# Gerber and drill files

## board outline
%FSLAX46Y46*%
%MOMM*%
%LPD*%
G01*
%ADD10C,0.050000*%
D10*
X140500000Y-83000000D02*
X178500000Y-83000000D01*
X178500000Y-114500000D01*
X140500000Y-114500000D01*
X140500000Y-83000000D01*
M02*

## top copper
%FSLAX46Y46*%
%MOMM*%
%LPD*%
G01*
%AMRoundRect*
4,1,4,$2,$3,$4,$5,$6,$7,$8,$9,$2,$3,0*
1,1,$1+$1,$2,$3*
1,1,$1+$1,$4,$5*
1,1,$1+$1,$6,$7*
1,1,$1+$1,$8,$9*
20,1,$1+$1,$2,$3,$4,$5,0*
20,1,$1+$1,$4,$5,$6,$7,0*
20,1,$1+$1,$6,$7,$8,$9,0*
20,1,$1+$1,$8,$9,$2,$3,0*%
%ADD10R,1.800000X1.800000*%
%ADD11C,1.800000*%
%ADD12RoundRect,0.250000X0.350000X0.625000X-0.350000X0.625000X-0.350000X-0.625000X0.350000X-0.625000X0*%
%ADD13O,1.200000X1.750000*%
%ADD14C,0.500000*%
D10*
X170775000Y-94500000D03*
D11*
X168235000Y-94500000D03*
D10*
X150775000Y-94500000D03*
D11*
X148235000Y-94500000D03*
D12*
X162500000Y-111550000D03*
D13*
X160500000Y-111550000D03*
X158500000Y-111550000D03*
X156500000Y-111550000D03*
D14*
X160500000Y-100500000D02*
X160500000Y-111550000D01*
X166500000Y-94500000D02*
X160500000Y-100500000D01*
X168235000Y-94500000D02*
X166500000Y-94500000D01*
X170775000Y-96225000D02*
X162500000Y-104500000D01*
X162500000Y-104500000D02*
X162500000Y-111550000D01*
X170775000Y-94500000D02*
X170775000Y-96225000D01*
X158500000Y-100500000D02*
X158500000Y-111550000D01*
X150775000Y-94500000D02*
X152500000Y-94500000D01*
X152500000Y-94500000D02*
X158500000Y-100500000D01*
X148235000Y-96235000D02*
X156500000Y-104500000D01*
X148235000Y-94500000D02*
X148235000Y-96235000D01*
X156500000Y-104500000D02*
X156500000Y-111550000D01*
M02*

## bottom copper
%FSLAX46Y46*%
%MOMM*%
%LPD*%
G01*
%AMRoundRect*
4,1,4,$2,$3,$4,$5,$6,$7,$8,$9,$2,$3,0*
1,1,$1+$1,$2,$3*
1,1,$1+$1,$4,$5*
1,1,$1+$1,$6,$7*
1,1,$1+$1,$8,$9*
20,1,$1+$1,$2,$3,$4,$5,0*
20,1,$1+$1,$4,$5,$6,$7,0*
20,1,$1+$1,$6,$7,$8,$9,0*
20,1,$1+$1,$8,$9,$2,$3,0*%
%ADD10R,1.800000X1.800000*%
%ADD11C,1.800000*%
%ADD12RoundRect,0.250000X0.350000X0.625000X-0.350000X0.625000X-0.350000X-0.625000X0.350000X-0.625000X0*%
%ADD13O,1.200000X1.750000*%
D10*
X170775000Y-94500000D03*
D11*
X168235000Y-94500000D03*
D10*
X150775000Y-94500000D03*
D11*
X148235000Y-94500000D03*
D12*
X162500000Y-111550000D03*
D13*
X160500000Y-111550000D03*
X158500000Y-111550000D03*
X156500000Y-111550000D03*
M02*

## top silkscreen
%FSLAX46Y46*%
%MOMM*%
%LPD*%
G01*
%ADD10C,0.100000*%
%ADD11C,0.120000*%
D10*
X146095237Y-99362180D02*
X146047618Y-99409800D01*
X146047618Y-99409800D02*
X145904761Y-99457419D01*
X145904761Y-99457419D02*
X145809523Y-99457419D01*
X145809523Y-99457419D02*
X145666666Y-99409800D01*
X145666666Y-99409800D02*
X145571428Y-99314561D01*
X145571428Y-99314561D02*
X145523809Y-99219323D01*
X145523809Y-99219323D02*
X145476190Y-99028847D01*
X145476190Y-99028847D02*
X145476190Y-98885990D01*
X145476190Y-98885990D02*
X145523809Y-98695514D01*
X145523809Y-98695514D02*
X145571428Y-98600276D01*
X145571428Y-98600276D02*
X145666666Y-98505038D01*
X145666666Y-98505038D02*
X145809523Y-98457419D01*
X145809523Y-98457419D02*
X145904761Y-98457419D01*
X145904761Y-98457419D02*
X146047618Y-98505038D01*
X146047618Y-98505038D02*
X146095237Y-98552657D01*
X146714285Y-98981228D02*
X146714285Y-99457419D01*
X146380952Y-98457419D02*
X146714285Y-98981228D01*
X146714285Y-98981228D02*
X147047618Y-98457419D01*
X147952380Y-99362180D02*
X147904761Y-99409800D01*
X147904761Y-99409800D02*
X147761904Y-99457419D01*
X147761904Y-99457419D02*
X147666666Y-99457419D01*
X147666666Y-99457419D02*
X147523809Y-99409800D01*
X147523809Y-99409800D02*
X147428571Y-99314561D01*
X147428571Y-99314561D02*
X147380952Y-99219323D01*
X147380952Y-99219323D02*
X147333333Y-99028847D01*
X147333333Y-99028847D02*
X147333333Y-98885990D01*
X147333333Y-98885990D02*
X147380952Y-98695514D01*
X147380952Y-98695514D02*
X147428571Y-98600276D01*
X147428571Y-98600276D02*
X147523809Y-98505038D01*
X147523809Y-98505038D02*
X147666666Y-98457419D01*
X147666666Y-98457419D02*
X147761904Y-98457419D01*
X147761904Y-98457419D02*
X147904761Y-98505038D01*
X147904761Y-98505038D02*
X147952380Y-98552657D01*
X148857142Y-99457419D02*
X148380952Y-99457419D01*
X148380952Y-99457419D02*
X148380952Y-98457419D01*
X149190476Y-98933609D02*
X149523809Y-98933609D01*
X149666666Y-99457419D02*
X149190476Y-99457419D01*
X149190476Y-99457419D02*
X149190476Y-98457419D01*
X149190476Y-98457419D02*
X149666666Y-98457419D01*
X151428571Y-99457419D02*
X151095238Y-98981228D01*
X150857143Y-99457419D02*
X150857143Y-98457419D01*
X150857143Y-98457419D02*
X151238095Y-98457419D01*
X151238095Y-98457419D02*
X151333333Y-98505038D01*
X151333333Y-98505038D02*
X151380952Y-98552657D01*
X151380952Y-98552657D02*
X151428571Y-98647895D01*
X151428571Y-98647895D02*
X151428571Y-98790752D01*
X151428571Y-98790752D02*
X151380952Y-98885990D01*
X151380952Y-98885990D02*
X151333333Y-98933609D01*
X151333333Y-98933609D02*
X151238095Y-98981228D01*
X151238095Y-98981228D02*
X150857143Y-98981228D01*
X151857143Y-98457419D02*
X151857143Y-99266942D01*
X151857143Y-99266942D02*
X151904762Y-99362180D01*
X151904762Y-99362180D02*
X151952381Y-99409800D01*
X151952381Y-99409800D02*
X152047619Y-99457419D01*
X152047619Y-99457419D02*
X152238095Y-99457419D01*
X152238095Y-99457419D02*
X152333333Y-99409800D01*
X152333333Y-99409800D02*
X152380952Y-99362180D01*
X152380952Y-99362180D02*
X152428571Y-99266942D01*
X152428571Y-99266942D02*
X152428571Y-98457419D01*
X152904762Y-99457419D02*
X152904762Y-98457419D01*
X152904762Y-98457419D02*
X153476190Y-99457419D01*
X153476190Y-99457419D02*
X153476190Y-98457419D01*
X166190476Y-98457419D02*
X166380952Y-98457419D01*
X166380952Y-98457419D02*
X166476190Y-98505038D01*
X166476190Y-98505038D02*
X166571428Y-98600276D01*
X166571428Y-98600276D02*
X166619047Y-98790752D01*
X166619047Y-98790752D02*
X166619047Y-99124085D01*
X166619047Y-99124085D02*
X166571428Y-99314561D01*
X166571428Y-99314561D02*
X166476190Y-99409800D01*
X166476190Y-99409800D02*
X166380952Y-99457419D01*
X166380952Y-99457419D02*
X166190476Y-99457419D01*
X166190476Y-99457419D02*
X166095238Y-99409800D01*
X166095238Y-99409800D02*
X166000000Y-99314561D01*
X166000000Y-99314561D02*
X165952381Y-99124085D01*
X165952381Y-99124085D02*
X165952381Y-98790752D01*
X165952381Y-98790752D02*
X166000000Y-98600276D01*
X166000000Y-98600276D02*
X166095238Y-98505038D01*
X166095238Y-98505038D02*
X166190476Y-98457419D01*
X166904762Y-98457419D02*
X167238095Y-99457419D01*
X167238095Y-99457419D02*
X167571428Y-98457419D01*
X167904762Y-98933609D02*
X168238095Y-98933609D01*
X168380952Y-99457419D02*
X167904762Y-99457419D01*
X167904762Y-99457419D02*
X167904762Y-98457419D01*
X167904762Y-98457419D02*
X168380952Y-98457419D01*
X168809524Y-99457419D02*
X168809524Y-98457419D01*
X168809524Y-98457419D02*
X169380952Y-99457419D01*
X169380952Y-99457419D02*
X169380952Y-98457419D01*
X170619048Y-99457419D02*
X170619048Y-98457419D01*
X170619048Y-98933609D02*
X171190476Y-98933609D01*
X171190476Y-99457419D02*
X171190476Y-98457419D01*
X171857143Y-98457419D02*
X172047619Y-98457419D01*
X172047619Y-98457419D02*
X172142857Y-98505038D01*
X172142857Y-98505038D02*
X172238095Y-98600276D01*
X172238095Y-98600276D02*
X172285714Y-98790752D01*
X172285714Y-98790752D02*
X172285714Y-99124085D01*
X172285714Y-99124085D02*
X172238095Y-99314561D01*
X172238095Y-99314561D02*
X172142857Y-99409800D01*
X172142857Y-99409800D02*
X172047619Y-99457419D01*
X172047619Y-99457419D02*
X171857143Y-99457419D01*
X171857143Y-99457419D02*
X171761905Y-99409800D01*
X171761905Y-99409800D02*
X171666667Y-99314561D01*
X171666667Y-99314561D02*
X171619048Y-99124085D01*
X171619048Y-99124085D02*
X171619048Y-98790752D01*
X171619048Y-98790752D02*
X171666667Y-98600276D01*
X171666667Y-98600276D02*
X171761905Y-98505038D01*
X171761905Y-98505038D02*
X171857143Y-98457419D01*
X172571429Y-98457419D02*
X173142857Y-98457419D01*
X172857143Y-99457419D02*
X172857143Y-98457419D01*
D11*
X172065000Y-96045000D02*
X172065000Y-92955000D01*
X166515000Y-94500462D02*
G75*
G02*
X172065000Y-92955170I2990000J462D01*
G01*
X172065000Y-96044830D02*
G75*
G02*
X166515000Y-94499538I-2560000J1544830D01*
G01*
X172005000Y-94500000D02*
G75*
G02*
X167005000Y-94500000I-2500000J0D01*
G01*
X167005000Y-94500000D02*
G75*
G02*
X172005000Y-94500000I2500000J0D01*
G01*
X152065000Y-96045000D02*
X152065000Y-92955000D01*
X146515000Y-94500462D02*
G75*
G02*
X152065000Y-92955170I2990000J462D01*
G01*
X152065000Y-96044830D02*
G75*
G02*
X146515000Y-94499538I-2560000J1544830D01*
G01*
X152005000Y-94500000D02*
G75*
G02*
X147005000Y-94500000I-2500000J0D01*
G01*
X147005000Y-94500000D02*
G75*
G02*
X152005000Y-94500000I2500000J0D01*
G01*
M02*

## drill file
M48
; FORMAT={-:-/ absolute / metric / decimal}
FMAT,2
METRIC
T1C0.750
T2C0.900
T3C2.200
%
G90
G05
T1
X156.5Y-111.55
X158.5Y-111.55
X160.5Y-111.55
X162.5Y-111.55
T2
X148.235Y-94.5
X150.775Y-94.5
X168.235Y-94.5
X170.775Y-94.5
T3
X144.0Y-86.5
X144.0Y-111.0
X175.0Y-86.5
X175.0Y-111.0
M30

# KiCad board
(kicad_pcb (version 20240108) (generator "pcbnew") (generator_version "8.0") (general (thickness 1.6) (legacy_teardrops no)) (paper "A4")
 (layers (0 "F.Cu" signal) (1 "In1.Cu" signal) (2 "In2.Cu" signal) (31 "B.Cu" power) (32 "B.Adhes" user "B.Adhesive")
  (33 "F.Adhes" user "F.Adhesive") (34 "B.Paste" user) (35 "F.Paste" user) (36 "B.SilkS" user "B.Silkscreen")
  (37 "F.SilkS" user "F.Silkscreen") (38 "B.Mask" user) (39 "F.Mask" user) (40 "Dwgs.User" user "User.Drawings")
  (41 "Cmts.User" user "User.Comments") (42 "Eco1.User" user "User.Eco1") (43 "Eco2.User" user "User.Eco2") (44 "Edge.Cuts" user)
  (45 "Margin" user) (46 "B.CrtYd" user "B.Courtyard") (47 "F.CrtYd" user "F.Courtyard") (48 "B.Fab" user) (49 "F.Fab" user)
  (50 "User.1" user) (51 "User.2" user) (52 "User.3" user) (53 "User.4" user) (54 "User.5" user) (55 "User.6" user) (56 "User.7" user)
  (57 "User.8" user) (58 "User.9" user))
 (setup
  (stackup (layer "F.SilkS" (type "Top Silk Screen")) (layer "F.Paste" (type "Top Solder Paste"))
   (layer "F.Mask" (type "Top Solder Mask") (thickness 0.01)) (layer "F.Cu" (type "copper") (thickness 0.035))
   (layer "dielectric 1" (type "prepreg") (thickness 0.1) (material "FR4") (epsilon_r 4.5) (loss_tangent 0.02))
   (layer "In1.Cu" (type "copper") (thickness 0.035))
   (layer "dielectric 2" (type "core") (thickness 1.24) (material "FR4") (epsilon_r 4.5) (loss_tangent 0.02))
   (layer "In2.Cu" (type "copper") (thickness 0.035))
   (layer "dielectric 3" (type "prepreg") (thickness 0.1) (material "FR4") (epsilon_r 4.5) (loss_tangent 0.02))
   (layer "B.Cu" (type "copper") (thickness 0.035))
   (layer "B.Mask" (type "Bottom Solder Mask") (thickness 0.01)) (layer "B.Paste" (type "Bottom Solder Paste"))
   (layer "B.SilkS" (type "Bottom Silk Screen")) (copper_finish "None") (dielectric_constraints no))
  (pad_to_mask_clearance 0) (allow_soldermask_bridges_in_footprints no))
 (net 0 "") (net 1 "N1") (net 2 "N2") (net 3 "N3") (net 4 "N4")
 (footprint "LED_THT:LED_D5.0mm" (layer "F.Cu") (at 170.775 94.5 180)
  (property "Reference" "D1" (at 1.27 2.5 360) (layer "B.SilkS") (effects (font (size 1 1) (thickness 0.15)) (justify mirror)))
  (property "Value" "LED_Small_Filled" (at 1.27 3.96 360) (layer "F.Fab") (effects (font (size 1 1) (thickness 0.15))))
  (fp_line (start -1.29 -1.545) (end -1.29 1.545) (stroke (width 0.12) (type solid)) (layer "F.SilkS"))
  (fp_arc (start 4.26 -0.000462) (mid 2.072002 2.880433) (end -1.29 1.54483) (stroke (width 0.12) (type solid)) (layer "F.SilkS"))
  (fp_arc (start -1.29 -1.54483) (mid 2.072002 -2.880433) (end 4.26 0.000462) (stroke (width 0.12) (type solid)) (layer "F.SilkS"))
  (fp_circle (center 1.27 0) (end 3.77 0) (stroke (width 0.12) (type solid)) (fill none) (layer "F.SilkS"))
  (pad "1" thru_hole rect (at 0 0 180) (size 1.8 1.8) (drill 0.9) (layers "*.Cu" "*.Mask") (remove_unused_layers no) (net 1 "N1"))
  (pad "2" thru_hole circle (at 2.54 0 180) (size 1.8 1.8) (drill 0.9) (layers "*.Cu" "*.Mask") (remove_unused_layers no) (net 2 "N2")))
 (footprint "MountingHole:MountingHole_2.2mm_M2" (layer "F.Cu") (at 175 86.5)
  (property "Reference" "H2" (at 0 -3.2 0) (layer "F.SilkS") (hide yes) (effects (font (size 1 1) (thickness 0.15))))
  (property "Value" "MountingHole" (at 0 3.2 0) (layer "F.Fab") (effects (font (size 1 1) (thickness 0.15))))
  (pad "" np_thru_hole circle (at 0 0) (size 2.2 2.2) (drill 2.2) (layers "*.Cu" "*.Mask")))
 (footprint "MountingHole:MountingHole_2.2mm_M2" (layer "F.Cu") (at 144 111)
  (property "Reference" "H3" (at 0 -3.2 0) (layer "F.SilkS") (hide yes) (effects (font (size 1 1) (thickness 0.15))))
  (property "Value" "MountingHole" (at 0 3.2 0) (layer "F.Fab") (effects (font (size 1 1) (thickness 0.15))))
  (pad "" np_thru_hole circle (at 0 0) (size 2.2 2.2) (drill 2.2) (layers "*.Cu" "*.Mask")))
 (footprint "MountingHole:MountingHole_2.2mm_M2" (layer "F.Cu") (at 144 86.5)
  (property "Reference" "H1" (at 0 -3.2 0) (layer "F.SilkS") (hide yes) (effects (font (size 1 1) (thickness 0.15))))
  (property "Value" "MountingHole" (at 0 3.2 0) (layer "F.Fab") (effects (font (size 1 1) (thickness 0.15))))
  (pad "" np_thru_hole circle (at 0 0) (size 2.2 2.2) (drill 2.2) (layers "*.Cu" "*.Mask")))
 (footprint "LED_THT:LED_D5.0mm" (layer "F.Cu") (at 150.775 94.5 180)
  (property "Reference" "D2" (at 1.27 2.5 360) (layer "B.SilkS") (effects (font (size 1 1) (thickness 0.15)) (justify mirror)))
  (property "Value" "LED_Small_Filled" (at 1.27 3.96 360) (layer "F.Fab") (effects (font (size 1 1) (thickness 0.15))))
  (fp_line (start -1.29 -1.545) (end -1.29 1.545) (stroke (width 0.12) (type solid)) (layer "F.SilkS"))
  (fp_arc (start 4.26 -0.000462) (mid 2.072002 2.880433) (end -1.29 1.54483) (stroke (width 0.12) (type solid)) (layer "F.SilkS"))
  (fp_arc (start -1.29 -1.54483) (mid 2.072002 -2.880433) (end 4.26 0.000462) (stroke (width 0.12) (type solid)) (layer "F.SilkS"))
  (fp_circle (center 1.27 0) (end 3.77 0) (stroke (width 0.12) (type solid)) (fill none) (layer "F.SilkS"))
  (pad "1" thru_hole rect (at 0 0 180) (size 1.8 1.8) (drill 0.9) (layers "*.Cu" "*.Mask") (remove_unused_layers no) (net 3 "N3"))
  (pad "2" thru_hole circle (at 2.54 0 180) (size 1.8 1.8) (drill 0.9) (layers "*.Cu" "*.Mask") (remove_unused_layers no) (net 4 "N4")))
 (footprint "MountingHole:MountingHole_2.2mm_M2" (layer "F.Cu") (at 175 111)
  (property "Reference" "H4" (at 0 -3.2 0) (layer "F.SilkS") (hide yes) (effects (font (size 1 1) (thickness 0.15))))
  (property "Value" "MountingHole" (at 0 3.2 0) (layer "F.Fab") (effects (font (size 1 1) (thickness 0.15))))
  (pad "" np_thru_hole circle (at 0 0) (size 2.2 2.2) (drill 2.2) (layers "*.Cu" "*.Mask")))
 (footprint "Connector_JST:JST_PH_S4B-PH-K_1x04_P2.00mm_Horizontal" (layer "B.Cu") (at 162.5 111.55 180)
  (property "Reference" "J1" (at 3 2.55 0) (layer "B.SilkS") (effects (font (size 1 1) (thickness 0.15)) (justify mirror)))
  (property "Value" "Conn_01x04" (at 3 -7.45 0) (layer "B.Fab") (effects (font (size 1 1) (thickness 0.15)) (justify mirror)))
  (pad "1" thru_hole roundrect (at 0 0 180) (size 1.2 1.75) (drill 0.75) (layers "*.Cu" "*.Mask") (remove_unused_layers no)
   (roundrect_rratio 0.208333) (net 1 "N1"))
  (pad "2" thru_hole oval (at 2 0 180) (size 1.2 1.75) (drill 0.75) (layers "*.Cu" "*.Mask") (remove_unused_layers no) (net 2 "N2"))
  (pad "3" thru_hole oval (at 4 0 180) (size 1.2 1.75) (drill 0.75) (layers "*.Cu" "*.Mask") (remove_unused_layers no) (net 3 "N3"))
  (pad "4" thru_hole oval (at 6 0 180) (size 1.2 1.75) (drill 0.75) (layers "*.Cu" "*.Mask") (remove_unused_layers no) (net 4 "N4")))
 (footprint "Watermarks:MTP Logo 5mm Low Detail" (layer "B.Cu") (at 154 104.5 180)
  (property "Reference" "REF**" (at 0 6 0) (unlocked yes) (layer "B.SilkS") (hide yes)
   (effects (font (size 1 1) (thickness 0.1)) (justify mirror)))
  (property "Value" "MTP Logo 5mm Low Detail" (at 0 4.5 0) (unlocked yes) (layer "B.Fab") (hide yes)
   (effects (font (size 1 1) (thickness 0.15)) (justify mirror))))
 (gr_rect (start 140.5 83) (end 178.5 114.5) (stroke (width 0.05) (type default)) (fill none) (layer "Edge.Cuts"))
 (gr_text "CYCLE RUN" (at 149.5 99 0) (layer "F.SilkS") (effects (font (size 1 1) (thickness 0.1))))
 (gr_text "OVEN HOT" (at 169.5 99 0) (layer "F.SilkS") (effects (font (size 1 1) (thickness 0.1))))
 (segment (start 160.5 100.5) (end 160.5 111.55) (width 0.5) (layer "F.Cu") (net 2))
 (segment (start 166.5 94.5) (end 160.5 100.5) (width 0.5) (layer "F.Cu") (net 2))
 (segment (start 168.235 94.5) (end 166.5 94.5) (width 0.5) (layer "F.Cu") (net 2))
 (segment (start 170.775 96.225) (end 162.5 104.5) (width 0.5) (layer "F.Cu") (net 1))
 (segment (start 162.5 104.5) (end 162.5 111.55) (width 0.5) (layer "F.Cu") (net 1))
 (segment (start 170.775 94.5) (end 170.775 96.225) (width 0.5) (layer "F.Cu") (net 1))
 (segment (start 158.5 100.5) (end 158.5 111.55) (width 0.5) (layer "F.Cu") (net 3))
 (segment (start 150.775 94.5) (end 152.5 94.5) (width 0.5) (layer "F.Cu") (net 3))
 (segment (start 152.5 94.5) (end 158.5 100.5) (width 0.5) (layer "F.Cu") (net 3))
 (segment (start 148.235 96.235) (end 156.5 104.5) (width 0.5) (layer "F.Cu") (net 4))
 (segment (start 148.235 94.5) (end 148.235 96.235) (width 0.5) (layer "F.Cu") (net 4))
 (segment (start 156.5 104.5) (end 156.5 111.55) (width 0.5) (layer "F.Cu") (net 4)))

